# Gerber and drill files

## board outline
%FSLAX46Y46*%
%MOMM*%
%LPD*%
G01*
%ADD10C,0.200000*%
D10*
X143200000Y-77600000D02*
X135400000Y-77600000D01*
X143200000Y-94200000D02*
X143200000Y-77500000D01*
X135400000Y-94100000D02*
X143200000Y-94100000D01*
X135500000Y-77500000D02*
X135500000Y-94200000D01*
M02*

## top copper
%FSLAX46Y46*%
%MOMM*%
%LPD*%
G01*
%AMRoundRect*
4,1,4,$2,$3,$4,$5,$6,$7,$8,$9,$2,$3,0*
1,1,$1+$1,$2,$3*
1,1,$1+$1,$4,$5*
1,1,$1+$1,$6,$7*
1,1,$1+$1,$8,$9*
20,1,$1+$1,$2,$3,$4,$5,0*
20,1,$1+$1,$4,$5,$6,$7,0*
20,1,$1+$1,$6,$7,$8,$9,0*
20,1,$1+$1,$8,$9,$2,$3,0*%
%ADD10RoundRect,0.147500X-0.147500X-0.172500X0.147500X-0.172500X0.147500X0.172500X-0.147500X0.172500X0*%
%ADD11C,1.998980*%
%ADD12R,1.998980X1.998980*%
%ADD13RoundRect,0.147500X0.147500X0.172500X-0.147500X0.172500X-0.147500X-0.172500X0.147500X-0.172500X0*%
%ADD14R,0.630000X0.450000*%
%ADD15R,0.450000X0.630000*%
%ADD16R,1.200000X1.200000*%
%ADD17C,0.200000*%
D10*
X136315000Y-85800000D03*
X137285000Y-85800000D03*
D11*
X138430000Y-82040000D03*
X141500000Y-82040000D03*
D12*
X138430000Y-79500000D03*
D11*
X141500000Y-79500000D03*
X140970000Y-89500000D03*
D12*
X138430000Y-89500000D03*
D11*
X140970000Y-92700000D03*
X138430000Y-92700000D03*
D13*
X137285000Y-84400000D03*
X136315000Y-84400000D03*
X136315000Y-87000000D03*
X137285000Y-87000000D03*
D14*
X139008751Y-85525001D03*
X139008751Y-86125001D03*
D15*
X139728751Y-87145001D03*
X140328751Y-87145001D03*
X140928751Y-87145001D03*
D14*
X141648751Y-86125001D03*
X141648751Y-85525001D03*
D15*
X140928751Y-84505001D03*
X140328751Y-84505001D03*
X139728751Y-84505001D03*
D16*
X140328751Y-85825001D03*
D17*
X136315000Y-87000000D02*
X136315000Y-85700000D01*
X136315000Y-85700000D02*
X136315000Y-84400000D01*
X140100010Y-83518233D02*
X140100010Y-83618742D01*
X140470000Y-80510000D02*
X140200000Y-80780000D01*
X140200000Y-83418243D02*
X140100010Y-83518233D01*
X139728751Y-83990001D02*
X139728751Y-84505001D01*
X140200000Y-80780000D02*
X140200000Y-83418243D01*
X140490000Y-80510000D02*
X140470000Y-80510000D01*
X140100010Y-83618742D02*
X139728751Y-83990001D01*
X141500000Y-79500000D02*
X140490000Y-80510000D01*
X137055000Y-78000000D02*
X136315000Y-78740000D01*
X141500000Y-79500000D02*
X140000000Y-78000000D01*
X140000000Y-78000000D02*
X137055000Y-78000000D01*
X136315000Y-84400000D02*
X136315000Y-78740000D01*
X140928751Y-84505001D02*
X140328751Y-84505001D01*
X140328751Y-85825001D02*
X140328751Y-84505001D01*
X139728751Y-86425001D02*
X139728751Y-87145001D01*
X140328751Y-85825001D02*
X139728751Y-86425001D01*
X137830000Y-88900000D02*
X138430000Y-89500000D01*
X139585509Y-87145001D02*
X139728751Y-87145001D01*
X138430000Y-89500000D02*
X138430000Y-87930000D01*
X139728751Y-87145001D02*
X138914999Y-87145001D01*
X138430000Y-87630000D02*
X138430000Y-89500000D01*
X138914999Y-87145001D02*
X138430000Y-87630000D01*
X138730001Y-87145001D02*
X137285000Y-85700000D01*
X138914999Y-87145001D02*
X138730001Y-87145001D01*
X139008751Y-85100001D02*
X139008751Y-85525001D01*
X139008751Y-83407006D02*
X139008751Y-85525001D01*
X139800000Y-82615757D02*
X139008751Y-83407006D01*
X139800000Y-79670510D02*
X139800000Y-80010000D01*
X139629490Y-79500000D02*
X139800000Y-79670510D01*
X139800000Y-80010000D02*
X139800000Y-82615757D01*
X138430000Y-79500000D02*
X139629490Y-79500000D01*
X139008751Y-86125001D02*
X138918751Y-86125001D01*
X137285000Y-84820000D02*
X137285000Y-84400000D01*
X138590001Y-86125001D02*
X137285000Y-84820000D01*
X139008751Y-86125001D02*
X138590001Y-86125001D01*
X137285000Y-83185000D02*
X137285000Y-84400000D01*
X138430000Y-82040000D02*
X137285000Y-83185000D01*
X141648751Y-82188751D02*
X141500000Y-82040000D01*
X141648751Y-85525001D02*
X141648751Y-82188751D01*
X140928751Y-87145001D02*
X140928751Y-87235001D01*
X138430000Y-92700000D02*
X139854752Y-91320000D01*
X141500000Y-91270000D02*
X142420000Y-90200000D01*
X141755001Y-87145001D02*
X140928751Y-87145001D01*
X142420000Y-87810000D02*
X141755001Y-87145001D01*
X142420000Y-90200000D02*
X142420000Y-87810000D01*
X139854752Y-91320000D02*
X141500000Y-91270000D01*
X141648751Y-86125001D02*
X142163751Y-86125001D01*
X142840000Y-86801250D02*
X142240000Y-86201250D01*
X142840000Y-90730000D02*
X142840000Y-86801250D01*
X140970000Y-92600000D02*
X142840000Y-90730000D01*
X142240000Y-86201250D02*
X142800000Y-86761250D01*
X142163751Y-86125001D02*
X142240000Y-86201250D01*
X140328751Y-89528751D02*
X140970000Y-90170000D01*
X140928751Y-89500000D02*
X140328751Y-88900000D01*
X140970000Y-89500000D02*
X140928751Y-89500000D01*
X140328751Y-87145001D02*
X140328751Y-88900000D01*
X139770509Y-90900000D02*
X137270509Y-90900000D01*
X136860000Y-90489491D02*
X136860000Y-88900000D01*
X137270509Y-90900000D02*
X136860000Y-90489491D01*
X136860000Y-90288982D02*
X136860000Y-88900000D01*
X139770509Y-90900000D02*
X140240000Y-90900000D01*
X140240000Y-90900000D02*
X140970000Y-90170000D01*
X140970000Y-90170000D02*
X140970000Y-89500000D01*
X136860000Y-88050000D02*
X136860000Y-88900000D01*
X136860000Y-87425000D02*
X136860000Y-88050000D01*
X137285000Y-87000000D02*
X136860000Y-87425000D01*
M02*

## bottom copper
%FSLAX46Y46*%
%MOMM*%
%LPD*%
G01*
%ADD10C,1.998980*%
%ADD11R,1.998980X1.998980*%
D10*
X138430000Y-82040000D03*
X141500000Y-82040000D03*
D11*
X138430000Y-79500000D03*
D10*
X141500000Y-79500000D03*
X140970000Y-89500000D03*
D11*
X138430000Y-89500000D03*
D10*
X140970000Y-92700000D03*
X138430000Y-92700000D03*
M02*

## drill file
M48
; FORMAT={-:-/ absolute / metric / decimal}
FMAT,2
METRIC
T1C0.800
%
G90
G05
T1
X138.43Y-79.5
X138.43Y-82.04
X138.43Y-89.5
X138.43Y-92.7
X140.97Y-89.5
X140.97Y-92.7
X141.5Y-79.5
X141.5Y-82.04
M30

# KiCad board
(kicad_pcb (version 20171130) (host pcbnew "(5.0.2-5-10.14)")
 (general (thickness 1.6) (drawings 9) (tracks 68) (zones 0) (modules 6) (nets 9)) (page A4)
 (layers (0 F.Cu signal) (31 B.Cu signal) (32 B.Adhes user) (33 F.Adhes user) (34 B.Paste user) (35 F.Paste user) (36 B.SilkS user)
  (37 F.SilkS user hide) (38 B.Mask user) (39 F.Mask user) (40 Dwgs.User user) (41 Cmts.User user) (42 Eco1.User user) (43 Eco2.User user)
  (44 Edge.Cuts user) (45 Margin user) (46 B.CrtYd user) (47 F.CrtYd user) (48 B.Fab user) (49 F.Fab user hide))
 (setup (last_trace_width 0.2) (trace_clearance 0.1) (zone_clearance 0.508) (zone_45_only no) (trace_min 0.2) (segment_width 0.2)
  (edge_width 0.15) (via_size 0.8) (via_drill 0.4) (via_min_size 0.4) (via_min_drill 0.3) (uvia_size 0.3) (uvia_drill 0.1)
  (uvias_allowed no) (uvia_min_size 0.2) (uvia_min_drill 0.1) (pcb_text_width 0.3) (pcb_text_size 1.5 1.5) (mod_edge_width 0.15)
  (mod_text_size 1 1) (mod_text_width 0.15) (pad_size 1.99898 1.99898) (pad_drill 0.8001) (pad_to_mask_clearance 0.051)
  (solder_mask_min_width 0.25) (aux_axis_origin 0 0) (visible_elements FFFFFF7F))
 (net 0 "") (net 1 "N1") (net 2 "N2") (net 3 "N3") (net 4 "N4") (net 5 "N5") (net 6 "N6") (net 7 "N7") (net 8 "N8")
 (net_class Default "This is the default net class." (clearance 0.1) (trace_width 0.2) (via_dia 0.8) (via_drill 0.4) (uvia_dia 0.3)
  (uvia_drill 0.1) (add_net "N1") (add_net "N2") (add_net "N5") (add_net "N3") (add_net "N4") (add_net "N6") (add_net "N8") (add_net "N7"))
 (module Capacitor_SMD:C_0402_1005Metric (layer F.Cu) (at 136.8 85.8)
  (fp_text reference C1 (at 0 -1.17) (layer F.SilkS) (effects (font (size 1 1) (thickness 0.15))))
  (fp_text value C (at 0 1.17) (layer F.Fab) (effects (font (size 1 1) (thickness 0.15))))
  (pad 1 smd roundrect (at -0.485 0) (size 0.59 0.64) (layers F.Cu F.Paste F.Mask) (roundrect_rratio 0.25) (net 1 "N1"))
  (pad 2 smd roundrect (at 0.485 0) (size 0.59 0.64) (layers F.Cu F.Paste F.Mask) (roundrect_rratio 0.25) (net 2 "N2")))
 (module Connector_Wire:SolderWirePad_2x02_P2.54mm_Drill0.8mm (layer F.Cu) (at 138.43 79.5)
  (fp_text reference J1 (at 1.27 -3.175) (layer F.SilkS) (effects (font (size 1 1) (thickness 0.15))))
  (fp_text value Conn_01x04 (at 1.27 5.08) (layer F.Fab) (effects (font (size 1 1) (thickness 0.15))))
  (pad 3 thru_hole circle (at 0 2.54) (size 1.99898 1.99898) (drill 0.8001) (layers *.Cu *.Mask) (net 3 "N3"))
  (pad 4 thru_hole circle (at 3.07 2.54) (size 1.99898 1.99898) (drill 0.8001) (layers *.Cu *.Mask) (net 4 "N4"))
  (pad 1 thru_hole rect (at 0 0) (size 1.99898 1.99898) (drill 0.8001) (layers *.Cu *.Mask) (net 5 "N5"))
  (pad 2 thru_hole circle (at 3.07 0) (size 1.99898 1.99898) (drill 0.8001) (layers *.Cu *.Mask) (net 1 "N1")))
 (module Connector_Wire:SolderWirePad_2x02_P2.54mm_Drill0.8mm (layer F.Cu) (at 138.43 89.5)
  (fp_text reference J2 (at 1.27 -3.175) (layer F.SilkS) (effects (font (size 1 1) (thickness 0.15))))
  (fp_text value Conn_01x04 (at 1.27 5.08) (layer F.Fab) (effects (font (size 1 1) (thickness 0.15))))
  (pad 2 thru_hole circle (at 2.54 0) (size 1.99898 1.99898) (drill 0.8001) (layers *.Cu *.Mask) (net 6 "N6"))
  (pad 1 thru_hole rect (at 0 0) (size 1.99898 1.99898) (drill 0.8001) (layers *.Cu *.Mask) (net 2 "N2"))
  (pad 4 thru_hole circle (at 2.54 3.2) (size 1.99898 1.99898) (drill 0.8001) (layers *.Cu *.Mask) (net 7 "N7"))
  (pad 3 thru_hole circle (at 0 3.2) (size 1.99898 1.99898) (drill 0.8001) (layers *.Cu *.Mask) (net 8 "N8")))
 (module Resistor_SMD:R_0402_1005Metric (layer F.Cu) (at 136.8 84.4 180)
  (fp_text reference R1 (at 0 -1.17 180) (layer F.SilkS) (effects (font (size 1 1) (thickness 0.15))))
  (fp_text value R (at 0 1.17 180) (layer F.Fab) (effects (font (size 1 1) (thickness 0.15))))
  (pad 1 smd roundrect (at -0.485 0 180) (size 0.59 0.64) (layers F.Cu F.Paste F.Mask) (roundrect_rratio 0.25) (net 3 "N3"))
  (pad 2 smd roundrect (at 0.485 0 180) (size 0.59 0.64) (layers F.Cu F.Paste F.Mask) (roundrect_rratio 0.25) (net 1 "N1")))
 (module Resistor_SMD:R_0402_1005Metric (layer F.Cu) (at 136.8 87 180)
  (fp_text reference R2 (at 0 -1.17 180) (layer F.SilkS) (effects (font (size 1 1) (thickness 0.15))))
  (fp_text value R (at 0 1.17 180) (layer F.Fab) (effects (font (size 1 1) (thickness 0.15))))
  (pad 2 smd roundrect (at 0.485 0 180) (size 0.59 0.64) (layers F.Cu F.Paste F.Mask) (roundrect_rratio 0.25) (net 1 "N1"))
  (pad 1 smd roundrect (at -0.485 0 180) (size 0.59 0.64) (layers F.Cu F.Paste F.Mask) (roundrect_rratio 0.25) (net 6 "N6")))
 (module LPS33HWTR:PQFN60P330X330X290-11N (layer F.Cu) (at 140.328751 85.825001)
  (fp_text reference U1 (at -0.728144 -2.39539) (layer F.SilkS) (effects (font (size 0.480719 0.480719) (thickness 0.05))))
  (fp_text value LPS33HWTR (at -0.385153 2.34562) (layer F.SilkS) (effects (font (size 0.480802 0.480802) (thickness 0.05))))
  (pad 1 smd rect (at -1.32 -0.3) (size 0.63 0.45) (layers F.Cu F.Paste F.Mask) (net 5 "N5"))
  (pad 2 smd rect (at -1.32 0.3) (size 0.63 0.45) (layers F.Cu F.Paste F.Mask) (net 3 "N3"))
  (pad 3 smd rect (at -0.6 1.32 90) (size 0.63 0.45) (layers F.Cu F.Paste F.Mask) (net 2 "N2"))
  (pad 4 smd rect (at 0 1.32 90) (size 0.63 0.45) (layers F.Cu F.Paste F.Mask) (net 6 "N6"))
  (pad 5 smd rect (at 0.6 1.32 90) (size 0.63 0.45) (layers F.Cu F.Paste F.Mask) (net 8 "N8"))
  (pad 6 smd rect (at 1.32 0.3 180) (size 0.63 0.45) (layers F.Cu F.Paste F.Mask) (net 7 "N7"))
  (pad 7 smd rect (at 1.32 -0.3 180) (size 0.63 0.45) (layers F.Cu F.Paste F.Mask) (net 4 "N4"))
  (pad 8 smd rect (at 0.6 -1.32 270) (size 0.63 0.45) (layers F.Cu F.Paste F.Mask) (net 2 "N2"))
  (pad 9 smd rect (at 0 -1.32 270) (size 0.63 0.45) (layers F.Cu F.Paste F.Mask) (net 2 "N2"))
  (pad 10 smd rect (at -0.6 -1.32 270) (size 0.63 0.45) (layers F.Cu F.Paste F.Mask) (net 1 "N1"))
  (pad EP smd rect (at 0 0) (size 1.2 1.2) (layers F.Cu F.Paste F.Mask) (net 2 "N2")))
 (gr_line (start 143.2 77.6) (end 135.4 77.6) (layer Edge.Cuts) (width 0.2))
 (gr_line (start 143.2 94.2) (end 143.2 77.5) (layer Edge.Cuts) (width 0.2))
 (gr_line (start 135.4 94.1) (end 143.2 94.1) (layer Edge.Cuts) (width 0.2))
 (gr_line (start 135.5 77.5) (end 135.5 94.2) (layer Edge.Cuts) (width 0.2))
 (segment (start 136.315 87) (end 136.315 85.7) (width 0.2) (layer F.Cu) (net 1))
 (segment (start 136.315 85.7) (end 136.315 84.4) (width 0.2) (layer F.Cu) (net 1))
 (segment (start 140.10001 83.518233) (end 140.10001 83.618742) (width 0.2) (layer F.Cu) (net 1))
 (segment (start 140.47 80.51) (end 140.2 80.78) (width 0.2) (layer F.Cu) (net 1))
 (segment (start 140.2 83.418243) (end 140.10001 83.518233) (width 0.2) (layer F.Cu) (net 1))
 (segment (start 139.728751 83.990001) (end 139.728751 84.505001) (width 0.2) (layer F.Cu) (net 1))
 (segment (start 140.2 80.78) (end 140.2 83.418243) (width 0.2) (layer F.Cu) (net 1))
 (segment (start 140.49 80.51) (end 140.47 80.51) (width 0.2) (layer F.Cu) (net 1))
 (segment (start 140.10001 83.618742) (end 139.728751 83.990001) (width 0.2) (layer F.Cu) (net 1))
 (segment (start 141.5 79.5) (end 140.49 80.51) (width 0.2) (layer F.Cu) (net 1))
 (segment (start 137.055 78) (end 136.315 78.74) (width 0.2) (layer F.Cu) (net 1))
 (segment (start 141.5 79.5) (end 140 78) (width 0.2) (layer F.Cu) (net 1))
 (segment (start 140 78) (end 137.055 78) (width 0.2) (layer F.Cu) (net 1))
 (segment (start 136.315 84.4) (end 136.315 78.74) (width 0.2) (layer F.Cu) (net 1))
 (segment (start 140.928751 84.505001) (end 140.328751 84.505001) (width 0.2) (layer F.Cu) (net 2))
 (segment (start 140.328751 85.825001) (end 140.328751 84.505001) (width 0.2) (layer F.Cu) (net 2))
 (segment (start 139.728751 86.425001) (end 139.728751 87.145001) (width 0.2) (layer F.Cu) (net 2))
 (segment (start 140.328751 85.825001) (end 139.728751 86.425001) (width 0.2) (layer F.Cu) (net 2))
 (segment (start 137.83 88.9) (end 138.43 89.5) (width 0.2) (layer F.Cu) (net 2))
 (segment (start 139.585509 87.145001) (end 139.728751 87.145001) (width 0.2) (layer F.Cu) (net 2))
 (segment (start 138.43 89.5) (end 138.43 87.93) (width 0.2) (layer F.Cu) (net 2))
 (segment (start 139.728751 87.145001) (end 138.914999 87.145001) (width 0.2) (layer F.Cu) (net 2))
 (segment (start 138.43 87.63) (end 138.43 89.5) (width 0.2) (layer F.Cu) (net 2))
 (segment (start 138.914999 87.145001) (end 138.43 87.63) (width 0.2) (layer F.Cu) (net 2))
 (segment (start 138.730001 87.145001) (end 137.285 85.7) (width 0.2) (layer F.Cu) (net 2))
 (segment (start 138.914999 87.145001) (end 138.730001 87.145001) (width 0.2) (layer F.Cu) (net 2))
 (segment (start 139.008751 85.100001) (end 139.008751 85.525001) (width 0.2) (layer F.Cu) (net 5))
 (segment (start 139.008751 83.407006) (end 139.008751 85.525001) (width 0.2) (layer F.Cu) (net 5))
 (segment (start 139.8 82.615757) (end 139.008751 83.407006) (width 0.2) (layer F.Cu) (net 5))
 (segment (start 139.8 79.67051) (end 139.8 80.01) (width 0.2) (layer F.Cu) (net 5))
 (segment (start 139.62949 79.5) (end 139.8 79.67051) (width 0.2) (layer F.Cu) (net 5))
 (segment (start 139.8 80.01) (end 139.8 82.615757) (width 0.2) (layer F.Cu) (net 5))
 (segment (start 138.43 79.5) (end 139.62949 79.5) (width 0.2) (layer F.Cu) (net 5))
 (segment (start 139.008751 86.125001) (end 138.918751 86.125001) (width 0.2) (layer F.Cu) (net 3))
 (segment (start 137.285 84.82) (end 137.285 84.4) (width 0.2) (layer F.Cu) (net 3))
 (segment (start 138.590001 86.125001) (end 137.285 84.82) (width 0.2) (layer F.Cu) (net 3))
 (segment (start 139.008751 86.125001) (end 138.590001 86.125001) (width 0.2) (layer F.Cu) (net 3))
 (segment (start 137.285 83.185) (end 137.285 84.4) (width 0.2) (layer F.Cu) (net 3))
 (segment (start 138.43 82.04) (end 137.285 83.185) (width 0.2) (layer F.Cu) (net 3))
 (segment (start 141.648751 82.188751) (end 141.5 82.04) (width 0.2) (layer F.Cu) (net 4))
 (segment (start 141.648751 85.525001) (end 141.648751 82.188751) (width 0.2) (layer F.Cu) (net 4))
 (segment (start 140.928751 87.145001) (end 140.928751 87.235001) (width 0.2) (layer F.Cu) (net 8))
 (segment (start 138.43 92.7) (end 139.854752 91.32) (width 0.2) (layer F.Cu) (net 8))
 (segment (start 141.5 91.27) (end 142.42 90.2) (width 0.2) (layer F.Cu) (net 8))
 (segment (start 141.755001 87.145001) (end 140.928751 87.145001) (width 0.2) (layer F.Cu) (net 8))
 (segment (start 142.42 87.81) (end 141.755001 87.145001) (width 0.2) (layer F.Cu) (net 8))
 (segment (start 142.42 90.2) (end 142.42 87.81) (width 0.2) (layer F.Cu) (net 8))
 (segment (start 139.854752 91.32) (end 141.5 91.27) (width 0.2) (layer F.Cu) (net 8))
 (segment (start 141.648751 86.125001) (end 142.163751 86.125001) (width 0.2) (layer F.Cu) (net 7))
 (segment (start 142.84 86.80125) (end 142.24 86.20125) (width 0.2) (layer F.Cu) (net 7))
 (segment (start 142.84 90.73) (end 142.84 86.80125) (width 0.2) (layer F.Cu) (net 7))
 (segment (start 140.97 92.6) (end 142.84 90.73) (width 0.2) (layer F.Cu) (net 7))
 (segment (start 142.24 86.20125) (end 142.8 86.76125) (width 0.2) (layer F.Cu) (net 7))
 (segment (start 142.163751 86.125001) (end 142.24 86.20125) (width 0.2) (layer F.Cu) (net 7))
 (segment (start 140.328751 89.528751) (end 140.97 90.17) (width 0.2) (layer F.Cu) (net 6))
 (segment (start 140.928751 89.5) (end 140.328751 88.9) (width 0.2) (layer F.Cu) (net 6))
 (segment (start 140.97 89.5) (end 140.928751 89.5) (width 0.2) (layer F.Cu) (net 6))
 (segment (start 140.328751 87.145001) (end 140.328751 88.9) (width 0.2) (layer F.Cu) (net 6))
 (segment (start 139.770509 90.9) (end 137.270509 90.9) (width 0.2) (layer F.Cu) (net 6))
 (segment (start 136.86 90.489491) (end 136.86 88.9) (width 0.2) (layer F.Cu) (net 6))
 (segment (start 137.270509 90.9) (end 136.86 90.489491) (width 0.2) (layer F.Cu) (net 6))
 (segment (start 136.86 90.288982) (end 136.86 88.9) (width 0.2) (layer F.Cu) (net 6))
 (segment (start 139.770509 90.9) (end 140.24 90.9) (width 0.2) (layer F.Cu) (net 6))
 (segment (start 140.24 90.9) (end 140.97 90.17) (width 0.2) (layer F.Cu) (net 6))
 (segment (start 140.97 90.17) (end 140.97 89.5) (width 0.2) (layer F.Cu) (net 6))
 (segment (start 136.86 88.05) (end 136.86 88.9) (width 0.2) (layer F.Cu) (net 6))
 (segment (start 136.86 87.425) (end 136.86 88.05) (width 0.2) (layer F.Cu) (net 6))
 (segment (start 137.285 87) (end 136.86 87.425) (width 0.2) (layer F.Cu) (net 6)))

